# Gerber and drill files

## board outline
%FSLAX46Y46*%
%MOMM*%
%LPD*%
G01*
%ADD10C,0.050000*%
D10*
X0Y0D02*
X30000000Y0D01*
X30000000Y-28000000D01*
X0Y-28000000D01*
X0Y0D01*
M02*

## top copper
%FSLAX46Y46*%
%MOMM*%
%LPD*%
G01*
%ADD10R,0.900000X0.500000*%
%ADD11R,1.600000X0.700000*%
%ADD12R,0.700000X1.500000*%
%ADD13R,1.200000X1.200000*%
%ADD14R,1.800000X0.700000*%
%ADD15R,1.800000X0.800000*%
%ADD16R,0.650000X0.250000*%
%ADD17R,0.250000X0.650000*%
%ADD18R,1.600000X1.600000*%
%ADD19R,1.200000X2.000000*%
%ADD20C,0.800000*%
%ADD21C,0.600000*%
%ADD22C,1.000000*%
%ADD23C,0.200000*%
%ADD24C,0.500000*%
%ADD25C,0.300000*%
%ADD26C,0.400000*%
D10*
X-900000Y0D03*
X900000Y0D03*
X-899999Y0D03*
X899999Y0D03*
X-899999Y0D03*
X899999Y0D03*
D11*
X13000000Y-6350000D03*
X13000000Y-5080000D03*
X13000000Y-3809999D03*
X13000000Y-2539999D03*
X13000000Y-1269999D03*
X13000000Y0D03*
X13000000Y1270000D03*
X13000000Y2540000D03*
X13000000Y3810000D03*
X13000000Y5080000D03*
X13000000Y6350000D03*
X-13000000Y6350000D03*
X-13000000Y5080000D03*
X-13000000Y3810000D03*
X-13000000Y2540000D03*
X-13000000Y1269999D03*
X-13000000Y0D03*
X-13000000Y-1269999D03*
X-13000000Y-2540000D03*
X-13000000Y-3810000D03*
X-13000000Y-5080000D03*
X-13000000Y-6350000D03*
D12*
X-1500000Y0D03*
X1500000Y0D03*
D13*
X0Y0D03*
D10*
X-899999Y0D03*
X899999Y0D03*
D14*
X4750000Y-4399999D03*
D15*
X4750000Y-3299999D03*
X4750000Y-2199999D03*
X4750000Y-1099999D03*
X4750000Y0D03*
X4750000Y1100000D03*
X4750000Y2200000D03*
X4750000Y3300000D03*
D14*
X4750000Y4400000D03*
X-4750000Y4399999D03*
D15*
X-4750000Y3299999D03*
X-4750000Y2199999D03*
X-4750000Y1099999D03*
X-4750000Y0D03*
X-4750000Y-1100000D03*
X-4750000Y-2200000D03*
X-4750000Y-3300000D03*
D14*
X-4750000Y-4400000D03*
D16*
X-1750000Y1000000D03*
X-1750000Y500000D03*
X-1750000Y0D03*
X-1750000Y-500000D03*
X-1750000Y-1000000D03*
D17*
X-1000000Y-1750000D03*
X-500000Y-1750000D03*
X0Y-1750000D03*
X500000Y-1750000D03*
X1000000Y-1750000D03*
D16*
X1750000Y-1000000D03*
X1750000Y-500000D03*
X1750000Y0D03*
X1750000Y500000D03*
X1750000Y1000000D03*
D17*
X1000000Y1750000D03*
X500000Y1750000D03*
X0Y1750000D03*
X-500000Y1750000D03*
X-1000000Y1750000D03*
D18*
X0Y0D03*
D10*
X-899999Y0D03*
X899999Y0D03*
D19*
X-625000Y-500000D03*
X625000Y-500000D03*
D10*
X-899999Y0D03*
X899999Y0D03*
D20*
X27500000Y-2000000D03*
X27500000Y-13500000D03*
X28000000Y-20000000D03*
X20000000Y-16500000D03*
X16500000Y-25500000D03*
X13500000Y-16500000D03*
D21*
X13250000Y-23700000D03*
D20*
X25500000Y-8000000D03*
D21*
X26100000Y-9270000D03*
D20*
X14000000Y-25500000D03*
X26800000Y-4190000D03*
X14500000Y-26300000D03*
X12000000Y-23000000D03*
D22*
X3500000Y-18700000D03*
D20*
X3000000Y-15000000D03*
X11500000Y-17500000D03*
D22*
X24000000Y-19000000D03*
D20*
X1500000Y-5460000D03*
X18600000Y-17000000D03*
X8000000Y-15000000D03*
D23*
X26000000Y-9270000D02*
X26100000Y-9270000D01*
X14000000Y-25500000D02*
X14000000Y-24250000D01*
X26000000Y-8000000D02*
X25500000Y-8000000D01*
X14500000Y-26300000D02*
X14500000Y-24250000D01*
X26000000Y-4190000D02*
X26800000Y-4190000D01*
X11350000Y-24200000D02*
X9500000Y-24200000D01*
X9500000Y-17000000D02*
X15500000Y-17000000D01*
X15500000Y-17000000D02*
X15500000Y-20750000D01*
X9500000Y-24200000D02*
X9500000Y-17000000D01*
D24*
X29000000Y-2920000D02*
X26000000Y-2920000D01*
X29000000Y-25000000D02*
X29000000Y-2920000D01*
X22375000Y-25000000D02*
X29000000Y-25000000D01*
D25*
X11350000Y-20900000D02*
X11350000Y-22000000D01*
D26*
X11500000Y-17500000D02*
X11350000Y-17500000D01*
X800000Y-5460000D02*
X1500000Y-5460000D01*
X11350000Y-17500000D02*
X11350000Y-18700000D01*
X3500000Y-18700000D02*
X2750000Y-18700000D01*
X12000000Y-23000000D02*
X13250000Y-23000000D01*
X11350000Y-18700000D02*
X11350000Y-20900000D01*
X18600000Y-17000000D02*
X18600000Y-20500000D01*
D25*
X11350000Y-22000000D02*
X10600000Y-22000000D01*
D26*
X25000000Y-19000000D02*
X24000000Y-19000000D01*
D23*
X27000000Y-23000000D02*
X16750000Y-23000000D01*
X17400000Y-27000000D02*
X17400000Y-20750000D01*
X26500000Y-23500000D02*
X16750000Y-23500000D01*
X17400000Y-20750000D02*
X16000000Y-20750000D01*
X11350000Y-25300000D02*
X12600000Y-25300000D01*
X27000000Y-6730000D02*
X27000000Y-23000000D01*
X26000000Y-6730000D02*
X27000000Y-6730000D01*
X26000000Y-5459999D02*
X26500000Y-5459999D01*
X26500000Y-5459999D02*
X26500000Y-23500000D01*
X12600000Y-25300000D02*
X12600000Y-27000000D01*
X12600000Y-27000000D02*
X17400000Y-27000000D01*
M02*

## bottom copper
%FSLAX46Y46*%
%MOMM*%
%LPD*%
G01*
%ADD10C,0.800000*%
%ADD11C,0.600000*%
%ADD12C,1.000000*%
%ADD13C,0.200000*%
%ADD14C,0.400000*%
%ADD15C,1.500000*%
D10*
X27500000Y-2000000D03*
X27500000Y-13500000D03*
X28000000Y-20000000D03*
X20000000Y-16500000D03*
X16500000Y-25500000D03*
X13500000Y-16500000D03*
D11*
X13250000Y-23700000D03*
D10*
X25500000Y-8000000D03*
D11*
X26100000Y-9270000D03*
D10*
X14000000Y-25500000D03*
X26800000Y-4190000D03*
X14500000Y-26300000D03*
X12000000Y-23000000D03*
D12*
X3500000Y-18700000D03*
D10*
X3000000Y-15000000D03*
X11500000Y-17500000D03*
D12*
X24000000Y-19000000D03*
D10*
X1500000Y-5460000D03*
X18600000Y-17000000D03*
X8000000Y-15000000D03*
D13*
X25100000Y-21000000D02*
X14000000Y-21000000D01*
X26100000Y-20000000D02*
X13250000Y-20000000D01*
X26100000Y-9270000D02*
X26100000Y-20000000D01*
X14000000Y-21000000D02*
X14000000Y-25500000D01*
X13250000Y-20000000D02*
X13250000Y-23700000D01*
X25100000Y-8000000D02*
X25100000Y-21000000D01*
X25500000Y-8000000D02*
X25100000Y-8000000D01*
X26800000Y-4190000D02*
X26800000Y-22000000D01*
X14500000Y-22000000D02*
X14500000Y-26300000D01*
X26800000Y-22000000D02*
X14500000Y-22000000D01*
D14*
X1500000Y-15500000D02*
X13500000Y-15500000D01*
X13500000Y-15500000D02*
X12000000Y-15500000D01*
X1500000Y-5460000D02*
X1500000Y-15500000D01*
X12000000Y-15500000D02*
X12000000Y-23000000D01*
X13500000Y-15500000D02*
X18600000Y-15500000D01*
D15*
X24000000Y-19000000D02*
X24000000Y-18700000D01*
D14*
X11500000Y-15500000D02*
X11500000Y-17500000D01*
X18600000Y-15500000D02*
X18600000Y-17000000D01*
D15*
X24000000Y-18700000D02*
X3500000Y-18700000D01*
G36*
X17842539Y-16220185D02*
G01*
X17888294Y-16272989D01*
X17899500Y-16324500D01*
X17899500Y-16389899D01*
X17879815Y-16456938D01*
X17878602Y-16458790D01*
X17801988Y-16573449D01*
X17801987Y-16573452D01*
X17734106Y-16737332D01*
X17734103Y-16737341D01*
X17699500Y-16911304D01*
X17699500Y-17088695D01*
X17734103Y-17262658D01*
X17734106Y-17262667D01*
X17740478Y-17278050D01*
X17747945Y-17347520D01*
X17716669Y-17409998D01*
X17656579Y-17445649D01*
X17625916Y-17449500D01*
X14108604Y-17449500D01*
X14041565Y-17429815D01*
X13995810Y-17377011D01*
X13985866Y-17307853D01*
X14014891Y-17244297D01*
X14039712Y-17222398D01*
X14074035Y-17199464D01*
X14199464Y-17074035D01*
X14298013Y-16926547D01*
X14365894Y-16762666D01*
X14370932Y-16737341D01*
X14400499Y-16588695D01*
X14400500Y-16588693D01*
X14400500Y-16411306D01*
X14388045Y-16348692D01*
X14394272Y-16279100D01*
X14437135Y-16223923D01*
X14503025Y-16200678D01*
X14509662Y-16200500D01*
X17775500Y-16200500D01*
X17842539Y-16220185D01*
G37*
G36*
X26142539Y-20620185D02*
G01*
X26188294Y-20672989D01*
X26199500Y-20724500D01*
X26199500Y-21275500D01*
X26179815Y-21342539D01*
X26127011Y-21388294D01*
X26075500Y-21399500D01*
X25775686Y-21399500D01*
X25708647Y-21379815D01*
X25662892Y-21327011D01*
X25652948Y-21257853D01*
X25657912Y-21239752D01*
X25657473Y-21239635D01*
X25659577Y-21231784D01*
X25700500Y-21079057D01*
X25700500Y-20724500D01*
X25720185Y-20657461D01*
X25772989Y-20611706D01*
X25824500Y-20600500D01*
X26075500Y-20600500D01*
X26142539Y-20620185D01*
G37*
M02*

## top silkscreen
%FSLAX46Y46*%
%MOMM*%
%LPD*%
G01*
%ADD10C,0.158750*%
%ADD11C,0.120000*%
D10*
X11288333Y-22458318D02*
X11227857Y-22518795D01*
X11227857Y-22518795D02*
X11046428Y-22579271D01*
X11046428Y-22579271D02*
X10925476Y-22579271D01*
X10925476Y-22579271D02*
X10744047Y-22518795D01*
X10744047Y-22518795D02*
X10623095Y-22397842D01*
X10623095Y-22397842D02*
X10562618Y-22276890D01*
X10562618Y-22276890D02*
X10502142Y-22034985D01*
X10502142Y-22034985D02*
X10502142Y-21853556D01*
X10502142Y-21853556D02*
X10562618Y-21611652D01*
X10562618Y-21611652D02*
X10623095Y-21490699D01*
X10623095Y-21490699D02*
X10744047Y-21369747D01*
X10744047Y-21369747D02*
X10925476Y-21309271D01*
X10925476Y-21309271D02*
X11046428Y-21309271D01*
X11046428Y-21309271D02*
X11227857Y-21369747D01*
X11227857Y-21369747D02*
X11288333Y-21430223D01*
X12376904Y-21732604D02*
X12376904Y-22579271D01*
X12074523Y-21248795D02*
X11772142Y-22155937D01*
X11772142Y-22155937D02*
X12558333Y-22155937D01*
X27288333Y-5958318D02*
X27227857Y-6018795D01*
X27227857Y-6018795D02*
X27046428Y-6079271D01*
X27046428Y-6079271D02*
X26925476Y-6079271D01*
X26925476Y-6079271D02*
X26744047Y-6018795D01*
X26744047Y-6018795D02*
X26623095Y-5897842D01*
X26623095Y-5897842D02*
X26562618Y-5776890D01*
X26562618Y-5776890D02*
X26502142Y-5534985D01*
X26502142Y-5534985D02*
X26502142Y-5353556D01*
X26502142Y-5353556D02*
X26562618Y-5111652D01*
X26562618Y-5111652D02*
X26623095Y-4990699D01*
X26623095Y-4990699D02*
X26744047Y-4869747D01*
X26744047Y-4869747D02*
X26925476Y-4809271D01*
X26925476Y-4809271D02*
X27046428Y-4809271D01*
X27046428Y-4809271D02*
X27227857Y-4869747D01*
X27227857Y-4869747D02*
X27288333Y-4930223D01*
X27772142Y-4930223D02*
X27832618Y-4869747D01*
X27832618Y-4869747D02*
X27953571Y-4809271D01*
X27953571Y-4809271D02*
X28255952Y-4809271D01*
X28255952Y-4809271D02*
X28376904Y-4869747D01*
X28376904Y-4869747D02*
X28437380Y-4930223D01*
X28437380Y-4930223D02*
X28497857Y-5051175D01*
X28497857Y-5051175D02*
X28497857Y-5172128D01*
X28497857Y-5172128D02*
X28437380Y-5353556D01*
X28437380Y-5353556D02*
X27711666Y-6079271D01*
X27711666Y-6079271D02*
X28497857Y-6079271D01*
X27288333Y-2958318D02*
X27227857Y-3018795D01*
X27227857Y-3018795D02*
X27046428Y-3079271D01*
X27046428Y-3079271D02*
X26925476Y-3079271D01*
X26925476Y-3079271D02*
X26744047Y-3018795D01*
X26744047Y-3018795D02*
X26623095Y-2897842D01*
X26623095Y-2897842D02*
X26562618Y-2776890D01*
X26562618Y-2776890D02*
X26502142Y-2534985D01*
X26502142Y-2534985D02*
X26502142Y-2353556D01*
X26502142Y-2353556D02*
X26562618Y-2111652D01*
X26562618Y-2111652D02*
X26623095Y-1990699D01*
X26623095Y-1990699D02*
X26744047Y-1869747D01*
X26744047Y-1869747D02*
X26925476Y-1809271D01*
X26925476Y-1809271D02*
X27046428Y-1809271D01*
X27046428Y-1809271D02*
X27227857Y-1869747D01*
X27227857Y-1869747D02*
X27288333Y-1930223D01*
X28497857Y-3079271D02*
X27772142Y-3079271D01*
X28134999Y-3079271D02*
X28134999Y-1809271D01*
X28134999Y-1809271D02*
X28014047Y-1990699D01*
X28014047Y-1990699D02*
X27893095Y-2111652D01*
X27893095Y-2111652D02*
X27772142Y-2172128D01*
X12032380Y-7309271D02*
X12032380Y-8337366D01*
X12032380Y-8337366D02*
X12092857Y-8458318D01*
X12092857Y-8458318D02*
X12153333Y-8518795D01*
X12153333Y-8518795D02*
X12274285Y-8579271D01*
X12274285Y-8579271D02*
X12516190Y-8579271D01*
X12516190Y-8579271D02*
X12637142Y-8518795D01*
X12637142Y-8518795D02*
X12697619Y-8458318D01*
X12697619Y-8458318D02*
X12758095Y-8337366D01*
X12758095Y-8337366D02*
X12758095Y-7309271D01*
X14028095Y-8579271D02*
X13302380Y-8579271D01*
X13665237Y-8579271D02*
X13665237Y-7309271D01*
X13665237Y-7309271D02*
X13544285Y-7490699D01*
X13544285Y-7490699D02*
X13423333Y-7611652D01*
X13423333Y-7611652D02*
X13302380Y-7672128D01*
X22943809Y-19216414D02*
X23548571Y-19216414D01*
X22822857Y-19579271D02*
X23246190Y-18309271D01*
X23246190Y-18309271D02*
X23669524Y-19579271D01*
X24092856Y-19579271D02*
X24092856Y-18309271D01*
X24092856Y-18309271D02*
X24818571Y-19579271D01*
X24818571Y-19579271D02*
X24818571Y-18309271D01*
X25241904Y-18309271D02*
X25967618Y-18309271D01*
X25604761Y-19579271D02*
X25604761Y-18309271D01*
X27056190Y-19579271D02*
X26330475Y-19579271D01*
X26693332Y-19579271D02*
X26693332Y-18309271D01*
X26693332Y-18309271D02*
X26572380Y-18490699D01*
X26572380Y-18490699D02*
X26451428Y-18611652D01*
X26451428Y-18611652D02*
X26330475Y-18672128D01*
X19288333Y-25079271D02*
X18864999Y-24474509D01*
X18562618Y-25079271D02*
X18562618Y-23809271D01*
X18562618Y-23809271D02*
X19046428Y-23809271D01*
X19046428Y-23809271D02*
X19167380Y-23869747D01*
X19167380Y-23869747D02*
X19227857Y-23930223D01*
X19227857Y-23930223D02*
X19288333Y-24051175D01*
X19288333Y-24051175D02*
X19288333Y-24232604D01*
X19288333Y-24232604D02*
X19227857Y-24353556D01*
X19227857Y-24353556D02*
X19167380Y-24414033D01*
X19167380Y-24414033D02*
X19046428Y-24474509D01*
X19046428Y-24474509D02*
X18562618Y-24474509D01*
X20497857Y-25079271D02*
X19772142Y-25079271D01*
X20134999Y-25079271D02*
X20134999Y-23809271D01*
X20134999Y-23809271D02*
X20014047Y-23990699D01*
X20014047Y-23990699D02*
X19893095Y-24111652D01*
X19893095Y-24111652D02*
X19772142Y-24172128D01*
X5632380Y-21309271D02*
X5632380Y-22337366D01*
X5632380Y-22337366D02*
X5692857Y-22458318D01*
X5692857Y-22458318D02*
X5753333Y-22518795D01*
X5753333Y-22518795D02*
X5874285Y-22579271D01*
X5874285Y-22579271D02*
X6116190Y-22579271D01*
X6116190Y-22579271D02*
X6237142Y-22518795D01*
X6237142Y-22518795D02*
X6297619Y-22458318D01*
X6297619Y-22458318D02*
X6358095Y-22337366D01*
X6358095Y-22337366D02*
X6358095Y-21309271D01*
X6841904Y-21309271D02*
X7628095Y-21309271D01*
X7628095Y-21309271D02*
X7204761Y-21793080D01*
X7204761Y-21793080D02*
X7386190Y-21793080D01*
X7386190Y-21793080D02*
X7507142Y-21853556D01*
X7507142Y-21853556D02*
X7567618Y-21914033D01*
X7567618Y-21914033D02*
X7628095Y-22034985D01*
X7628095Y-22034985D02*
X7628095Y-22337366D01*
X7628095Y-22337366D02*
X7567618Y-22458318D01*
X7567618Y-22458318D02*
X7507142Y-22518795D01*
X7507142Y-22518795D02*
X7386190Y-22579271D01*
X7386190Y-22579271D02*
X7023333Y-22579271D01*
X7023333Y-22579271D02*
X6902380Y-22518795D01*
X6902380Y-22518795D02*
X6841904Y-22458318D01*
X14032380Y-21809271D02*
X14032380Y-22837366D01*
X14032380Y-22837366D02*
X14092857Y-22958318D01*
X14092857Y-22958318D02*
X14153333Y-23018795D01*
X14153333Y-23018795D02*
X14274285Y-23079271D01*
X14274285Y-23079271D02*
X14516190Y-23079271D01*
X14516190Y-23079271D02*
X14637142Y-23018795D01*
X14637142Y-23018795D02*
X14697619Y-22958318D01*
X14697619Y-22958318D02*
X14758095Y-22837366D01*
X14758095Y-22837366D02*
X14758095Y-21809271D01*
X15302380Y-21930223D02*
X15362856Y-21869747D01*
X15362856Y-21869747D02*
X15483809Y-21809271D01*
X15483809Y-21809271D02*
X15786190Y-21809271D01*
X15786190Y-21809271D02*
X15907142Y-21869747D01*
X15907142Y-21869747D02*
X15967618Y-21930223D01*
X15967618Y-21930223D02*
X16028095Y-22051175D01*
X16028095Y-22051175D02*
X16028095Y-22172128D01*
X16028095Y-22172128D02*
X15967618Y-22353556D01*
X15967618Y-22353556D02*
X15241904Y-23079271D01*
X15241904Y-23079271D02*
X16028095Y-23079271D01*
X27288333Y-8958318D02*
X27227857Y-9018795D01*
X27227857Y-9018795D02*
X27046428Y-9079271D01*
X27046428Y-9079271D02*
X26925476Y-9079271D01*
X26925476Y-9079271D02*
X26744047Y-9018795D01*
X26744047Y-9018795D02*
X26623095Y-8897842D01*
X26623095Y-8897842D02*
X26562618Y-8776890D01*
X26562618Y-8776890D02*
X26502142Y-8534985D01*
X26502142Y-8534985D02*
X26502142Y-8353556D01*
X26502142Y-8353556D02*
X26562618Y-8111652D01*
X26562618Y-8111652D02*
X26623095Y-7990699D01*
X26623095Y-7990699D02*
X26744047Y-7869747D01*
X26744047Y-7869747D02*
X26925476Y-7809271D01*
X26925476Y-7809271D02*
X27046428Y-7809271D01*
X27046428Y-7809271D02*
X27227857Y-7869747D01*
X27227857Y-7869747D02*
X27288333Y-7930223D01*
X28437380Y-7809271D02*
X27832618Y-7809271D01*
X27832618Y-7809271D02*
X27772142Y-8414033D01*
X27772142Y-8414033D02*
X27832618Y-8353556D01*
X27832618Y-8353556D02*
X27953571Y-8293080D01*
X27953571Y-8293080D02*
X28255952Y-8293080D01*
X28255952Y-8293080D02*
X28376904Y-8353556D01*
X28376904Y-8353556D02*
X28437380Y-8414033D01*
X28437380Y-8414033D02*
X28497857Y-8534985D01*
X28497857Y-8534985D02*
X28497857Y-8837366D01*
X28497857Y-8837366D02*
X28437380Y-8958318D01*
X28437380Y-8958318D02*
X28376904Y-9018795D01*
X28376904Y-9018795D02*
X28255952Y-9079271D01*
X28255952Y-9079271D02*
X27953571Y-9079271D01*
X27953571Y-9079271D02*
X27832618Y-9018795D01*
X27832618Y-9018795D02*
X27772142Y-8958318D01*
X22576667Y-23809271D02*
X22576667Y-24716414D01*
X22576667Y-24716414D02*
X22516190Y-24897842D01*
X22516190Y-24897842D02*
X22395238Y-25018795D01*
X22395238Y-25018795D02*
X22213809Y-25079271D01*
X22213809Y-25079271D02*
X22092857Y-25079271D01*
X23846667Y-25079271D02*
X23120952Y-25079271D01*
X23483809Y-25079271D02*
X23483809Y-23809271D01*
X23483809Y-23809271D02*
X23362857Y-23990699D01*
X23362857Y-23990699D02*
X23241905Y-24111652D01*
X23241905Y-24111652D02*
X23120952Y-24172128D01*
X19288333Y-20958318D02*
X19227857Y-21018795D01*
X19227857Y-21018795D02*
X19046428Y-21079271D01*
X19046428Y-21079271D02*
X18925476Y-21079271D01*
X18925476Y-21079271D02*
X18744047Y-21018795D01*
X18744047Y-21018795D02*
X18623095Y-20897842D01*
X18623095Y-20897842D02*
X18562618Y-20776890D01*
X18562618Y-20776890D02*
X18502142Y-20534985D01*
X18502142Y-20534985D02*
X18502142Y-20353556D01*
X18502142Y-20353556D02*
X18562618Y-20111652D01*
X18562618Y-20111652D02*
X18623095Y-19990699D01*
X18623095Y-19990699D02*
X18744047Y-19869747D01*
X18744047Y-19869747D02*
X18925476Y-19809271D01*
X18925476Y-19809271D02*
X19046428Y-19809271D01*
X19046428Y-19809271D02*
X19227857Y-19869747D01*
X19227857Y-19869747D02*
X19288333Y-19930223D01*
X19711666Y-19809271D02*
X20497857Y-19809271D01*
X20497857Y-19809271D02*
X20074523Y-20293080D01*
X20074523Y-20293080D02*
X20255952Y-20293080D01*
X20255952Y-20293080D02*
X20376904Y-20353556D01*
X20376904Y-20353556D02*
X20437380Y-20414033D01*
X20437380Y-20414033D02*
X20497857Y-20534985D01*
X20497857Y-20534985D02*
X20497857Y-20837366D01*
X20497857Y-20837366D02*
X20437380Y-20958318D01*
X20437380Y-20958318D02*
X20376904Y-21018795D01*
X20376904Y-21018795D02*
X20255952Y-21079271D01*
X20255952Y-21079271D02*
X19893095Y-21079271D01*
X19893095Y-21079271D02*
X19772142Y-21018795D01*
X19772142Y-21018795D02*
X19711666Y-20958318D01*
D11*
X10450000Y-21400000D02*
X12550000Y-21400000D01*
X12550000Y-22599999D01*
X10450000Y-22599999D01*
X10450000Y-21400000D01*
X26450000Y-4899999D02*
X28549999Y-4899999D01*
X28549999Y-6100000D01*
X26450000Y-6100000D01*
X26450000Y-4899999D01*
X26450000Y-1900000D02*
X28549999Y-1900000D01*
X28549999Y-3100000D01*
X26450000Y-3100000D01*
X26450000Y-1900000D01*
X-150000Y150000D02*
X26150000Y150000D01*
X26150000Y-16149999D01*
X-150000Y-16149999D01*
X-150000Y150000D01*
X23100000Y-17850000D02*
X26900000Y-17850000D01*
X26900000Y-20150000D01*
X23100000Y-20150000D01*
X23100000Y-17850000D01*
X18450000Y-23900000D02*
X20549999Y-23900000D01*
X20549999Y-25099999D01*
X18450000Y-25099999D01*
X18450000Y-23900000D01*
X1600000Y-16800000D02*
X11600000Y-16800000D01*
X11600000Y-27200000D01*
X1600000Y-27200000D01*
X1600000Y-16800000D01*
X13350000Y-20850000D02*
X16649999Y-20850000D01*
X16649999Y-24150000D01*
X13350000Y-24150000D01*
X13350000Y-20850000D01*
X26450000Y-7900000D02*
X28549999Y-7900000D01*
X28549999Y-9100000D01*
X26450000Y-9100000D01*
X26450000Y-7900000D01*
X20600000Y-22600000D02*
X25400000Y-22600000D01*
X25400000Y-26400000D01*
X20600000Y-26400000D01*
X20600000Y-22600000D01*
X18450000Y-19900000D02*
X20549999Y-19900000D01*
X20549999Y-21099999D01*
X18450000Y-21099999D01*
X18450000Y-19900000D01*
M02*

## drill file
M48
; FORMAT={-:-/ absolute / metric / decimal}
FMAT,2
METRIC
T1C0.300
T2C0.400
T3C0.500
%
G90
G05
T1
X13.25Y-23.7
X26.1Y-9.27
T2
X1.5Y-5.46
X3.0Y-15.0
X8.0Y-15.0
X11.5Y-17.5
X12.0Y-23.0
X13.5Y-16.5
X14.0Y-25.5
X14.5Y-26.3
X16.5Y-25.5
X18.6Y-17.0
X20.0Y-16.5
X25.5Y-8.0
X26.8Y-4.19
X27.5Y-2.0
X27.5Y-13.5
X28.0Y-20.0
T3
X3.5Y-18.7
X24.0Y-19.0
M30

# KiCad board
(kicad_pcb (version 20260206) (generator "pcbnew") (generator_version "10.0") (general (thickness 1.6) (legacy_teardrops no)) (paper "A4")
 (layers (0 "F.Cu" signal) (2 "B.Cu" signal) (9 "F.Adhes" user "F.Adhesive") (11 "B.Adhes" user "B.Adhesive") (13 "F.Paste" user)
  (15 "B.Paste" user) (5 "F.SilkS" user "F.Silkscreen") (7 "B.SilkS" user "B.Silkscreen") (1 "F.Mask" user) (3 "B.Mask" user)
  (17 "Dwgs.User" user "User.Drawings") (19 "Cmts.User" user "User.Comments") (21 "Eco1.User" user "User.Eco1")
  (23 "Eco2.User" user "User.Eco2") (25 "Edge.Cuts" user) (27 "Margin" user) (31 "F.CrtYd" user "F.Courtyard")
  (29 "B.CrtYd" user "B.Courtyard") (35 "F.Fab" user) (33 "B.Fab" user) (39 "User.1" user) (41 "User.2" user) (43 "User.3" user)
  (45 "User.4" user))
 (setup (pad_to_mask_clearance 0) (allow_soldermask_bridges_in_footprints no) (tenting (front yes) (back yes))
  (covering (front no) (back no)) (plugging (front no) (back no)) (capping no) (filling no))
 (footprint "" (layer "F.Cu") (at 11.5 22)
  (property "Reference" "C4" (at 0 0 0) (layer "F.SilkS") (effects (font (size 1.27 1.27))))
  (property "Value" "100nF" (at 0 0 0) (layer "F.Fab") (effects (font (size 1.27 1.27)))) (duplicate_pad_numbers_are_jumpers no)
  (fp_rect (start -1.05 -0.6) (end 1.05 0.599999) (stroke (width 0.12) (type default)) (fill no) (layer "F.SilkS"))
  (pad "1" smd rect (at -12.4 -22) (size 0.9 0.5) (layers "F.Cu" "F.Mask" "F.Paste") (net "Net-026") (thermal_bridge_angle 45))
  (pad "2" smd rect (at -10.6 -22) (size 0.9 0.5) (layers "F.Cu" "F.Mask" "F.Paste") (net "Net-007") (thermal_bridge_angle 45)))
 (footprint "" (layer "F.Cu") (at 27.5 5.5)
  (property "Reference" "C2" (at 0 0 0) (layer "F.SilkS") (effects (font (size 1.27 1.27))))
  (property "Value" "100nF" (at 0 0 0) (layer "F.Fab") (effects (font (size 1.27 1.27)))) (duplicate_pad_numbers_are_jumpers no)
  (fp_rect (start -1.05 -0.600001) (end 1.049999 0.6) (stroke (width 0.12) (type default)) (fill no) (layer "F.SilkS"))
  (pad "1" smd rect (at -28.399999 -5.5) (size 0.9 0.5) (layers "F.Cu" "F.Mask" "F.Paste") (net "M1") (thermal_bridge_angle 45))
  (pad "2" smd rect (at -26.600001 -5.5) (size 0.9 0.5) (layers "F.Cu" "F.Mask" "F.Paste") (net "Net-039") (thermal_bridge_angle 45)))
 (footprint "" (layer "F.Cu") (at 27.5 2.5)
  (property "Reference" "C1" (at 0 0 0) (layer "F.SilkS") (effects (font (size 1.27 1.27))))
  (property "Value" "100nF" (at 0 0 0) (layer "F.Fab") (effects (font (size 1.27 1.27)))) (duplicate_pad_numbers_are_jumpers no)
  (fp_rect (start -1.05 -0.6) (end 1.049999 0.6) (stroke (width 0.12) (type default)) (fill no) (layer "F.SilkS"))
  (pad "1" smd rect (at -28.399999 -2.5) (size 0.9 0.5) (layers "F.Cu" "F.Mask" "F.Paste") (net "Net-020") (thermal_bridge_angle 45))
  (pad "2" smd rect (at -26.600001 -2.5) (size 0.9 0.5) (layers "F.Cu" "F.Mask" "F.Paste") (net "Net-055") (thermal_bridge_angle 45)))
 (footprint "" (layer "F.Cu") (at 13 8)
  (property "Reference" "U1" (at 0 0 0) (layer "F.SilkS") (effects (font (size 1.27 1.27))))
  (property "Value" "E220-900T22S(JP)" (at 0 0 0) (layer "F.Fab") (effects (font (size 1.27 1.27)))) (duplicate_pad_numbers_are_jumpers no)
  (fp_rect (start -13.15 -8.15) (end 13.15 8.149999) (stroke (width 0.12) (type default)) (fill no) (layer "F.SilkS"))
  (pad "1" smd rect (at 0 -1.65) (size 1.6 0.7) (layers "F.Cu" "F.Mask" "F.Paste") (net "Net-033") (thermal_bridge_angle 45))
  (pad "2" smd rect (at 0 -2.92) (size 1.6 0.7) (layers "F.Cu" "F.Mask" "F.Paste") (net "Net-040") (thermal_bridge_angle 45))
  (pad "3" smd rect (at 0 -4.190001) (size 1.6 0.7) (layers "F.Cu" "F.Mask" "F.Paste") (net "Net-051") (thermal_bridge_angle 45))
  (pad "4" smd rect (at 0 -5.460001) (size 1.6 0.7) (layers "F.Cu" "F.Mask" "F.Paste") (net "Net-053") (thermal_bridge_angle 45))
  (pad "5" smd rect (at 0 -6.730001) (size 1.6 0.7) (layers "F.Cu" "F.Mask" "F.Paste") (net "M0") (thermal_bridge_angle 45))
  (pad "6" smd rect (at 0 -8) (size 1.6 0.7) (layers "F.Cu" "F.Mask" "F.Paste") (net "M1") (thermal_bridge_angle 45))
  (pad "7" smd rect (at 0 -9.27) (size 1.6 0.7) (layers "F.Cu" "F.Mask" "F.Paste") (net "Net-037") (thermal_bridge_angle 45))
  (pad "8" smd rect (at 0 -10.54) (size 1.6 0.7) (layers "F.Cu" "F.Mask" "F.Paste") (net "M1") (thermal_bridge_angle 45))
  (pad "9" smd rect (at 0 -11.81) (size 1.6 0.7) (layers "F.Cu" "F.Mask" "F.Paste") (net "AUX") (thermal_bridge_angle 45))
  (pad "10" smd rect (at 0 -13.08) (size 1.6 0.7) (layers "F.Cu" "F.Mask" "F.Paste") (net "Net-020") (thermal_bridge_angle 45))
  (pad "11" smd rect (at 0 -14.35) (size 1.6 0.7) (layers "F.Cu" "F.Mask" "F.Paste") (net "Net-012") (thermal_bridge_angle 45))
  (pad "12" smd rect (at -26 -14.35) (size 1.6 0.7) (layers "F.Cu" "F.Mask" "F.Paste") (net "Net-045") (thermal_bridge_angle 45))
  (pad "13" smd rect (at -26 -13.08) (size 1.6 0.7) (layers "F.Cu" "F.Mask" "F.Paste") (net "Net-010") (thermal_bridge_angle 45))
  (pad "14" smd rect (at -26 -11.81) (size 1.6 0.7) (layers "F.Cu" "F.Mask" "F.Paste") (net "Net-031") (thermal_bridge_angle 45))
  (pad "15" smd rect (at -26 -10.54) (size 1.6 0.7) (layers "F.Cu" "F.Mask" "F.Paste") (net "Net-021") (thermal_bridge_angle 45))
  (pad "16" smd rect (at -26 -9.269999) (size 1.6 0.7) (layers "F.Cu" "F.Mask" "F.Paste") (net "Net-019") (thermal_bridge_angle 45))
  (pad "17" smd rect (at -26 -8) (size 1.6 0.7) (layers "F.Cu" "F.Mask" "F.Paste") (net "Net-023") (thermal_bridge_angle 45))
  (pad "18" smd rect (at -26 -6.730001) (size 1.6 0.7) (layers "F.Cu" "F.Mask" "F.Paste") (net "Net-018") (thermal_bridge_angle 45))
  (pad "19" smd rect (at -26 -5.46) (size 1.6 0.7) (layers "F.Cu" "F.Mask" "F.Paste") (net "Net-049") (thermal_bridge_angle 45))
  (pad "20" smd rect (at -26 -4.19) (size 1.6 0.7) (layers "F.Cu" "F.Mask" "F.Paste") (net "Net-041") (thermal_bridge_angle 45))
  (pad "21" smd rect (at -26 -2.92) (size 1.6 0.7) (layers "F.Cu" "F.Mask" "F.Paste") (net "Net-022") (thermal_bridge_angle 45))
  (pad "22" smd rect (at -26 -1.65) (size 1.6 0.7) (layers "F.Cu" "F.Mask" "F.Paste") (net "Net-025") (thermal_bridge_angle 45)))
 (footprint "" (layer "F.Cu") (at 25 19)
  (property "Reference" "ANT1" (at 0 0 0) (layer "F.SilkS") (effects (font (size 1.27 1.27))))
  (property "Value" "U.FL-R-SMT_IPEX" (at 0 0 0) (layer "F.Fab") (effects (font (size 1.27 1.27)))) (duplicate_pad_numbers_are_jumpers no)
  (fp_rect (start -1.9 -1.15) (end 1.9 1.15) (stroke (width 0.12) (type default)) (fill no) (layer "F.SilkS"))
  (pad "G1" smd rect (at -26.5 -19) (size 0.7 1.5) (layers "F.Cu" "F.Mask" "F.Paste") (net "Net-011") (thermal_bridge_angle 45))
  (pad "G2" smd rect (at -23.5 -19) (size 0.7 1.5) (layers "F.Cu" "F.Mask" "F.Paste") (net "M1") (thermal_bridge_angle 45))
  (pad "S" smd rect (at -25 -19) (size 1.2 1.2) (layers "F.Cu" "F.Mask" "F.Paste") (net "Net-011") (thermal_bridge_angle 45)))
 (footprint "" (layer "F.Cu") (at 19.5 24.5)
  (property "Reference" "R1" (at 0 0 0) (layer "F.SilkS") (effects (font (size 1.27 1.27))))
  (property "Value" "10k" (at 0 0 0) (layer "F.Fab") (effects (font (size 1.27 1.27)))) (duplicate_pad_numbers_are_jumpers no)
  (fp_rect (start -1.05 -0.6) (end 1.049999 0.599999) (stroke (width 0.12) (type default)) (fill no) (layer "F.SilkS"))
  (pad "1" smd rect (at -20.399999 -24.5) (size 0.9 0.5) (layers "F.Cu" "F.Mask" "F.Paste") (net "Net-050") (thermal_bridge_angle 45))
  (pad "2" smd rect (at -18.600001 -24.5) (size 0.9 0.5) (layers "F.Cu" "F.Mask" "F.Paste") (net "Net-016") (thermal_bridge_angle 45)))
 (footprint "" (layer "F.Cu") (at 6.6 22)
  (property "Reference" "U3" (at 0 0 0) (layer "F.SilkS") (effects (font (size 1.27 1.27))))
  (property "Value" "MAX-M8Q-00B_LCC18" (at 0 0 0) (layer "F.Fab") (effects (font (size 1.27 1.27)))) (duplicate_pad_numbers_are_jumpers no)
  (fp_rect (start -5 -5.2) (end 5 5.2) (stroke (width 0.12) (type default)) (fill no) (layer "F.SilkS"))
  (pad "1" smd rect (at -1.85 -17.600001) (size 1.8 0.7) (layers "F.Cu" "F.Mask" "F.Paste") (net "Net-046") (thermal_bridge_angle 45))
  (pad "2" smd rect (at -1.85 -18.700001) (size 1.8 0.8) (layers "F.Cu" "F.Mask" "F.Paste") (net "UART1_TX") (thermal_bridge_angle 45))
  (pad "3" smd rect (at -1.85 -19.800001) (size 1.8 0.8) (layers "F.Cu" "F.Mask" "F.Paste") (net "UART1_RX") (thermal_bridge_angle 45))
  (pad "4" smd rect (at -1.85 -20.900001) (size 1.8 0.8) (layers "F.Cu" "F.Mask" "F.Paste") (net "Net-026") (thermal_bridge_angle 45))
  (pad "5" smd rect (at -1.85 -22) (size 1.8 0.8) (layers "F.Cu" "F.Mask" "F.Paste") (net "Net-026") (thermal_bridge_angle 45))
  (pad "6" smd rect (at -1.85 -23.1) (size 1.8 0.8) (layers "F.Cu" "F.Mask" "F.Paste") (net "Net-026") (thermal_bridge_angle 45))
  (pad "7" smd rect (at -1.85 -24.2) (size 1.8 0.8) (layers "F.Cu" "F.Mask" "F.Paste") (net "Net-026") (thermal_bridge_angle 45))
  (pad "8" smd rect (at -1.85 -25.3) (size 1.8 0.8) (layers "F.Cu" "F.Mask" "F.Paste") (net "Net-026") (thermal_bridge_angle 45))
  (pad "9" smd rect (at -1.85 -26.4) (size 1.8 0.7) (layers "F.Cu" "F.Mask" "F.Paste") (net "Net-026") (thermal_bridge_angle 45))
  (pad "10" smd rect (at -11.35 -26.399999) (size 1.8 0.7) (layers "F.Cu" "F.Mask" "F.Paste") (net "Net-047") (thermal_bridge_angle 45))
  (pad "11" smd rect (at -11.35 -25.299999) (size 1.8 0.8) (layers "F.Cu" "F.Mask" "F.Paste") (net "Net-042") (thermal_bridge_angle 45))
  (pad "12" smd rect (at -11.35 -24.199999) (size 1.8 0.8) (layers "F.Cu" "F.Mask" "F.Paste") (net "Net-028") (thermal_bridge_angle 45))
  (pad "13" smd rect (at -11.35 -23.099999) (size 1.8 0.8) (layers "F.Cu" "F.Mask" "F.Paste") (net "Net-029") (thermal_bridge_angle 45))
  (pad "14" smd rect (at -11.35 -22) (size 1.8 0.8) (layers "F.Cu" "F.Mask" "F.Paste") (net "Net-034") (thermal_bridge_angle 45))
  (pad "15" smd rect (at -11.35 -20.9) (size 1.8 0.8) (layers "F.Cu" "F.Mask" "F.Paste") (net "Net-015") (thermal_bridge_angle 45))
  (pad "16" smd rect (at -11.35 -19.8) (size 1.8 0.8) (layers "F.Cu" "F.Mask" "F.Paste") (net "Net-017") (thermal_bridge_angle 45))
  (pad "17" smd rect (at -11.35 -18.7) (size 1.8 0.8) (layers "F.Cu" "F.Mask" "F.Paste") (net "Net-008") (thermal_bridge_angle 45))
  (pad "18" smd rect (at -11.35 -17.6) (size 1.8 0.7) (layers "F.Cu" "F.Mask" "F.Paste") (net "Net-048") (thermal_bridge_angle 45)))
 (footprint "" (layer "F.Cu") (at 15 22.5)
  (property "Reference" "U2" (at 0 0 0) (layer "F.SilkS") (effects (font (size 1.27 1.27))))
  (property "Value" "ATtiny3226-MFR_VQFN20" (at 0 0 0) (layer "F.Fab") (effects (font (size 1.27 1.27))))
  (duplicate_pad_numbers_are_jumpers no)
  (fp_rect (start -1.65 -1.65) (end 1.649999 1.65) (stroke (width 0.12) (type default)) (fill no) (layer "F.SilkS"))
  (pad "1" smd rect (at -16.75 -23.5) (size 0.65 0.25) (layers "F.Cu" "F.Mask" "F.Paste") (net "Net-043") (thermal_bridge_angle 45))
  (pad "2" smd rect (at -16.75 -23) (size 0.65 0.25) (layers "F.Cu" "F.Mask" "F.Paste") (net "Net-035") (thermal_bridge_angle 45))
  (pad "3" smd rect (at -16.75 -22.5) (size 0.65 0.25) (layers "F.Cu" "F.Mask" "F.Paste") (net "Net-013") (thermal_bridge_angle 45))
  (pad "4" smd rect (at -16.75 -22) (size 0.65 0.25) (layers "F.Cu" "F.Mask" "F.Paste") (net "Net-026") (thermal_bridge_angle 45))
  (pad "5" smd rect (at -16.75 -21.5) (size 0.65 0.25) (layers "F.Cu" "F.Mask" "F.Paste") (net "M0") (thermal_bridge_angle 45))
  (pad "6" smd rect (at -16 -20.75) (size 0.25 0.65) (layers "F.Cu" "F.Mask" "F.Paste") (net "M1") (thermal_bridge_angle 45))
  (pad "7" smd rect (at -15.5 -20.75) (size 0.25 0.65) (layers "F.Cu" "F.Mask" "F.Paste") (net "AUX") (thermal_bridge_angle 45))
  (pad "8" smd rect (at -15 -20.75) (size 0.25 0.65) (layers "F.Cu" "F.Mask" "F.Paste") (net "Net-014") (thermal_bridge_angle 45))
  (pad "9" smd rect (at -14.5 -20.75) (size 0.25 0.65) (layers "F.Cu" "F.Mask" "F.Paste") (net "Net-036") (thermal_bridge_angle 45))
  (pad "10" smd rect (at -14 -20.75) (size 0.25 0.65) (layers "F.Cu" "F.Mask" "F.Paste") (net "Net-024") (thermal_bridge_angle 45))
  (pad "11" smd rect (at -13.25 -21.5) (size 0.65 0.25) (layers "F.Cu" "F.Mask" "F.Paste") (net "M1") (thermal_bridge_angle 45))
  (pad "12" smd rect (at -13.25 -22) (size 0.65 0.25) (layers "F.Cu" "F.Mask" "F.Paste") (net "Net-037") (thermal_bridge_angle 45))
  (pad "13" smd rect (at -13.25 -22.5) (size 0.65 0.25) (layers "F.Cu" "F.Mask" "F.Paste") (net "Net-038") (thermal_bridge_angle 45))
  (pad "14" smd rect (at -13.25 -23) (size 0.65 0.25) (layers "F.Cu" "F.Mask" "F.Paste") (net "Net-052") (thermal_bridge_angle 45))
  (pad "15" smd rect (at -13.25 -23.5) (size 0.65 0.25) (layers "F.Cu" "F.Mask" "F.Paste") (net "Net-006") (thermal_bridge_angle 45))
  (pad "16" smd rect (at -14 -24.25) (size 0.25 0.65) (layers "F.Cu" "F.Mask" "F.Paste") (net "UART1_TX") (thermal_bridge_angle 45))
  (pad "17" smd rect (at -14.5 -24.25) (size 0.25 0.65) (layers "F.Cu" "F.Mask" "F.Paste") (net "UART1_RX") (thermal_bridge_angle 45))
  (pad "18" smd rect (at -15 -24.25) (size 0.25 0.65) (layers "F.Cu" "F.Mask" "F.Paste") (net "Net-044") (thermal_bridge_angle 45))
  (pad "19" smd rect (at -15.5 -24.25) (size 0.25 0.65) (layers "F.Cu" "F.Mask" "F.Paste") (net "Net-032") (thermal_bridge_angle 45))
  (pad "20" smd rect (at -16 -24.25) (size 0.25 0.65) (layers "F.Cu" "F.Mask" "F.Paste") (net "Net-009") (thermal_bridge_angle 45))
  (pad "EP" smd rect (at -15 -22.5) (size 1.6 1.6) (layers "F.Cu" "F.Mask" "F.Paste") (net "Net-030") (thermal_bridge_angle 45)))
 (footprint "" (layer "F.Cu") (at 27.5 8.5)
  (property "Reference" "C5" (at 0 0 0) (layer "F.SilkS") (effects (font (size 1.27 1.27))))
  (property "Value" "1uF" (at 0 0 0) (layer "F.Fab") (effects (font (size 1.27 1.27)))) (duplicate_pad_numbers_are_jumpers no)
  (fp_rect (start -1.05 -0.6) (end 1.049999 0.6) (stroke (width 0.12) (type default)) (fill no) (layer "F.SilkS"))
  (pad "1" smd rect (at -28.399999 -8.5) (size 0.9 0.5) (layers "F.Cu" "F.Mask" "F.Paste") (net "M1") (thermal_bridge_angle 45))
  (pad "2" smd rect (at -26.600001 -8.5) (size 0.9 0.5) (layers "F.Cu" "F.Mask" "F.Paste") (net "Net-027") (thermal_bridge_angle 45)))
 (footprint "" (layer "F.Cu") (at 23 24.5)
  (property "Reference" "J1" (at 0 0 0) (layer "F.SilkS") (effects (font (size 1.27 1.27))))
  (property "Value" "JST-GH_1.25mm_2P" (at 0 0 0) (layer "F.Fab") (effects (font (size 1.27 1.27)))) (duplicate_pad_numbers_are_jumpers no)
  (fp_rect (start -2.4 -1.9) (end 2.4 1.9) (stroke (width 0.12) (type default)) (fill no) (layer "F.SilkS"))
  (pad "1" smd rect (at -23.625 -24) (size 1.2 2) (layers "F.Cu" "F.Mask" "F.Paste") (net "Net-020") (thermal_bridge_angle 45))
  (pad "2" smd rect (at -22.375 -24) (size 1.2 2) (layers "F.Cu" "F.Mask" "F.Paste") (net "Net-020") (thermal_bridge_angle 45)))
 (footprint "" (layer "F.Cu") (at 19.5 20.5)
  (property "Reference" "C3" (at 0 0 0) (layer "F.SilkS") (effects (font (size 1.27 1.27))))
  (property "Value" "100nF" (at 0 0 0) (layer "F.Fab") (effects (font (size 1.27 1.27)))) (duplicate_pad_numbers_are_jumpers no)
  (fp_rect (start -1.05 -0.6) (end 1.049999 0.599999) (stroke (width 0.12) (type default)) (fill no) (layer "F.SilkS"))
  (pad "1" smd rect (at -20.399999 -20.5) (size 0.9 0.5) (layers "F.Cu" "F.Mask" "F.Paste") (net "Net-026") (thermal_bridge_angle 45))
  (pad "2" smd rect (at -18.600001 -20.5) (size 0.9 0.5) (layers "F.Cu" "F.Mask" "F.Paste") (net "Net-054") (thermal_bridge_angle 45)))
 (gr_rect (start 0 0) (end 30 28) (stroke (width 0.05) (type default)) (fill no) (layer "Edge.Cuts"))
 (via (at 27.5 2) (size 0.8) (drill 0.4) (layers "F.Cu" "B.Cu") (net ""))
 (via (at 27.5 13.5) (size 0.8) (drill 0.4) (layers "F.Cu" "B.Cu") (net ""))
 (via (at 28 20) (size 0.8) (drill 0.4) (layers "F.Cu" "B.Cu") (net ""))
 (via (at 20 16.5) (size 0.8) (drill 0.4) (layers "F.Cu" "B.Cu") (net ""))
 (via (at 16.5 25.5) (size 0.8) (drill 0.4) (layers "F.Cu" "B.Cu") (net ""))
 (via (at 13.5 16.5) (size 0.8) (drill 0.4) (layers "F.Cu" "B.Cu") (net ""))
 (segment (start 26 9.27) (end 26.1 9.27) (width 0.2) (layer "F.Cu") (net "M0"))
 (segment (start 14 25.5) (end 14 24.25) (width 0.2) (layer "F.Cu") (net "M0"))
 (segment (start 26 8) (end 25.5 8) (width 0.2) (layer "F.Cu") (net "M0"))
 (via (at 13.25 23.7) (size 0.6) (drill 0.3) (layers "F.Cu" "B.Cu") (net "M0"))
 (via (at 25.5 8) (size 0.8) (drill 0.4) (layers "F.Cu" "B.Cu") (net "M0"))
 (via (at 26.1 9.27) (size 0.6) (drill 0.3) (layers "F.Cu" "B.Cu") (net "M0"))
 (via (at 14 25.5) (size 0.8) (drill 0.4) (layers "F.Cu" "B.Cu") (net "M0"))
 (segment (start 25.1 21) (end 14 21) (width 0.2) (layer "B.Cu") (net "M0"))
 (segment (start 26.1 20) (end 13.25 20) (width 0.2) (layer "B.Cu") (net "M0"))
 (segment (start 26.1 9.27) (end 26.1 20) (width 0.2) (layer "B.Cu") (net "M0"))
 (segment (start 14 21) (end 14 25.5) (width 0.2) (layer "B.Cu") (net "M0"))
 (segment (start 13.25 20) (end 13.25 23.7) (width 0.2) (layer "B.Cu") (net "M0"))
 (segment (start 25.1 8) (end 25.1 21) (width 0.2) (layer "B.Cu") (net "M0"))
 (segment (start 25.5 8) (end 25.1 8) (width 0.2) (layer "B.Cu") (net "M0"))
 (segment (start 14.5 26.3) (end 14.5 24.25) (width 0.2) (layer "F.Cu") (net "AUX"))
 (segment (start 26 4.19) (end 26.8 4.19) (width 0.2) (layer "F.Cu") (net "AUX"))
 (via (at 26.8 4.19) (size 0.8) (drill 0.4) (layers "F.Cu" "B.Cu") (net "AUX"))
 (via (at 14.5 26.3) (size 0.8) (drill 0.4) (layers "F.Cu" "B.Cu") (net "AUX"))
 (segment (start 26.8 4.19) (end 26.8 22) (width 0.2) (layer "B.Cu") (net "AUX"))
 (segment (start 14.5 22) (end 14.5 26.3) (width 0.2) (layer "B.Cu") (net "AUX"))
 (segment (start 26.8 22) (end 14.5 22) (width 0.2) (layer "B.Cu") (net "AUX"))
 (segment (start 11.35 24.2) (end 9.5 24.2) (width 0.2) (layer "F.Cu") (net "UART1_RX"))
 (segment (start 9.5 17) (end 15.5 17) (width 0.2) (layer "F.Cu") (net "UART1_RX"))
 (segment (start 15.5 17) (end 15.5 20.75) (width 0.2) (layer "F.Cu") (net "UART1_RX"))
 (segment (start 9.5 24.2) (end 9.5 17) (width 0.2) (layer "F.Cu") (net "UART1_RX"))
 (segment (start 29 2.92) (end 26 2.92) (width 0.5) (layer "F.Cu") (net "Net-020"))
 (segment (start 29 25) (end 29 2.92) (width 0.5) (layer "F.Cu") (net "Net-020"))
 (segment (start 22.375 25) (end 29 25) (width 0.5) (layer "F.Cu") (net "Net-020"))
 (segment (start 11.35 20.9) (end 11.35 22) (width 0.3) (layer "F.Cu") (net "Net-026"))
 (segment (start 11.5 17.5) (end 11.35 17.5) (width 0.4) (layer "F.Cu") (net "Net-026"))
 (segment (start 0.8 5.46) (end 1.5 5.46) (width 0.4) (layer "F.Cu") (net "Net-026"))
 (segment (start 11.35 17.5) (end 11.35 18.7) (width 0.4) (layer "F.Cu") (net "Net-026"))
 (segment (start 3.5 18.7) (end 2.75 18.7) (width 0.4) (layer "F.Cu") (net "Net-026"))
 (segment (start 12 23) (end 13.25 23) (width 0.4) (layer "F.Cu") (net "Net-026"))
 (segment (start 11.35 18.7) (end 11.35 20.9) (width 0.4) (layer "F.Cu") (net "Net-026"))
 (segment (start 18.6 17) (end 18.6 20.5) (width 0.4) (layer "F.Cu") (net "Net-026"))
 (segment (start 11.35 22) (end 10.6 22) (width 0.3) (layer "F.Cu") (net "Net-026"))
 (segment (start 25 19) (end 24 19) (width 0.4) (layer "F.Cu") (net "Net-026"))
 (via (at 12 23) (size 0.8) (drill 0.4) (layers "F.Cu" "B.Cu") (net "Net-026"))
 (via (at 3.5 18.7) (size 1) (drill 0.5) (layers "F.Cu" "B.Cu") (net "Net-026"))
 (via (at 3 15) (size 0.8) (drill 0.4) (layers "F.Cu" "B.Cu") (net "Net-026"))
 (via (at 11.5 17.5) (size 0.8) (drill 0.4) (layers "F.Cu" "B.Cu") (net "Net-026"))
 (via (at 24 19) (size 1) (drill 0.5) (layers "F.Cu" "B.Cu") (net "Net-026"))
 (via (at 1.5 5.46) (size 0.8) (drill 0.4) (layers "F.Cu" "B.Cu") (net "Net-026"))
 (via (at 18.6 17) (size 0.8) (drill 0.4) (layers "F.Cu" "B.Cu") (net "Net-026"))
 (via (at 8 15) (size 0.8) (drill 0.4) (layers "F.Cu" "B.Cu") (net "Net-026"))
 (segment (start 1.5 15.5) (end 13.5 15.5) (width 0.4) (layer "B.Cu") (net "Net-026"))
 (segment (start 13.5 15.5) (end 12 15.5) (width 0.4) (layer "B.Cu") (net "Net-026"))
 (segment (start 1.5 5.46) (end 1.5 15.5) (width 0.4) (layer "B.Cu") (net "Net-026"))
 (segment (start 12 15.5) (end 12 23) (width 0.4) (layer "B.Cu") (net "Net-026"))
 (segment (start 13.5 15.5) (end 18.6 15.5) (width 0.4) (layer "B.Cu") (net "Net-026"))
 (segment (start 24 19) (end 24 18.7) (width 1.5) (layer "B.Cu") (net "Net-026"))
 (segment (start 11.5 15.5) (end 11.5 17.5) (width 0.4) (layer "B.Cu") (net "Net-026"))
 (segment (start 18.6 15.5) (end 18.6 17) (width 0.4) (layer "B.Cu") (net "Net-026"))
 (segment (start 24 18.7) (end 3.5 18.7) (width 1.5) (layer "B.Cu") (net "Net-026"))
 (segment (start 27 23) (end 16.75 23) (width 0.2) (layer "F.Cu") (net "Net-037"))
 (segment (start 17.4 27) (end 17.4 20.75) (width 0.2) (layer "F.Cu") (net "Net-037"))
 (segment (start 26.5 23.5) (end 16.75 23.5) (width 0.2) (layer "F.Cu") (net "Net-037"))
 (segment (start 17.4 20.75) (end 16 20.75) (width 0.2) (layer "F.Cu") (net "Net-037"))
 (segment (start 11.35 25.3) (end 12.6 25.3) (width 0.2) (layer "F.Cu") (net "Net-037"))
 (segment (start 27 6.73) (end 27 23) (width 0.2) (layer "F.Cu") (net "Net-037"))
 (segment (start 26 6.73) (end 27 6.73) (width 0.2) (layer "F.Cu") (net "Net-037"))
 (segment (start 26 5.459999) (end 26.5 5.459999) (width 0.2) (layer "F.Cu") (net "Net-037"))
 (segment (start 26.5 5.459999) (end 26.5 23.5) (width 0.2) (layer "F.Cu") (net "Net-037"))
 (segment (start 12.6 25.3) (end 12.6 27) (width 0.2) (layer "F.Cu") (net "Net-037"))
 (segment (start 12.6 27) (end 17.4 27) (width 0.2) (layer "F.Cu") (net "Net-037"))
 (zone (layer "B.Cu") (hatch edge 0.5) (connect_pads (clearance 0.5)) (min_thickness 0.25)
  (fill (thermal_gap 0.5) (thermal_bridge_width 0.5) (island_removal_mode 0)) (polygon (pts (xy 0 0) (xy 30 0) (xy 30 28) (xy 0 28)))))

